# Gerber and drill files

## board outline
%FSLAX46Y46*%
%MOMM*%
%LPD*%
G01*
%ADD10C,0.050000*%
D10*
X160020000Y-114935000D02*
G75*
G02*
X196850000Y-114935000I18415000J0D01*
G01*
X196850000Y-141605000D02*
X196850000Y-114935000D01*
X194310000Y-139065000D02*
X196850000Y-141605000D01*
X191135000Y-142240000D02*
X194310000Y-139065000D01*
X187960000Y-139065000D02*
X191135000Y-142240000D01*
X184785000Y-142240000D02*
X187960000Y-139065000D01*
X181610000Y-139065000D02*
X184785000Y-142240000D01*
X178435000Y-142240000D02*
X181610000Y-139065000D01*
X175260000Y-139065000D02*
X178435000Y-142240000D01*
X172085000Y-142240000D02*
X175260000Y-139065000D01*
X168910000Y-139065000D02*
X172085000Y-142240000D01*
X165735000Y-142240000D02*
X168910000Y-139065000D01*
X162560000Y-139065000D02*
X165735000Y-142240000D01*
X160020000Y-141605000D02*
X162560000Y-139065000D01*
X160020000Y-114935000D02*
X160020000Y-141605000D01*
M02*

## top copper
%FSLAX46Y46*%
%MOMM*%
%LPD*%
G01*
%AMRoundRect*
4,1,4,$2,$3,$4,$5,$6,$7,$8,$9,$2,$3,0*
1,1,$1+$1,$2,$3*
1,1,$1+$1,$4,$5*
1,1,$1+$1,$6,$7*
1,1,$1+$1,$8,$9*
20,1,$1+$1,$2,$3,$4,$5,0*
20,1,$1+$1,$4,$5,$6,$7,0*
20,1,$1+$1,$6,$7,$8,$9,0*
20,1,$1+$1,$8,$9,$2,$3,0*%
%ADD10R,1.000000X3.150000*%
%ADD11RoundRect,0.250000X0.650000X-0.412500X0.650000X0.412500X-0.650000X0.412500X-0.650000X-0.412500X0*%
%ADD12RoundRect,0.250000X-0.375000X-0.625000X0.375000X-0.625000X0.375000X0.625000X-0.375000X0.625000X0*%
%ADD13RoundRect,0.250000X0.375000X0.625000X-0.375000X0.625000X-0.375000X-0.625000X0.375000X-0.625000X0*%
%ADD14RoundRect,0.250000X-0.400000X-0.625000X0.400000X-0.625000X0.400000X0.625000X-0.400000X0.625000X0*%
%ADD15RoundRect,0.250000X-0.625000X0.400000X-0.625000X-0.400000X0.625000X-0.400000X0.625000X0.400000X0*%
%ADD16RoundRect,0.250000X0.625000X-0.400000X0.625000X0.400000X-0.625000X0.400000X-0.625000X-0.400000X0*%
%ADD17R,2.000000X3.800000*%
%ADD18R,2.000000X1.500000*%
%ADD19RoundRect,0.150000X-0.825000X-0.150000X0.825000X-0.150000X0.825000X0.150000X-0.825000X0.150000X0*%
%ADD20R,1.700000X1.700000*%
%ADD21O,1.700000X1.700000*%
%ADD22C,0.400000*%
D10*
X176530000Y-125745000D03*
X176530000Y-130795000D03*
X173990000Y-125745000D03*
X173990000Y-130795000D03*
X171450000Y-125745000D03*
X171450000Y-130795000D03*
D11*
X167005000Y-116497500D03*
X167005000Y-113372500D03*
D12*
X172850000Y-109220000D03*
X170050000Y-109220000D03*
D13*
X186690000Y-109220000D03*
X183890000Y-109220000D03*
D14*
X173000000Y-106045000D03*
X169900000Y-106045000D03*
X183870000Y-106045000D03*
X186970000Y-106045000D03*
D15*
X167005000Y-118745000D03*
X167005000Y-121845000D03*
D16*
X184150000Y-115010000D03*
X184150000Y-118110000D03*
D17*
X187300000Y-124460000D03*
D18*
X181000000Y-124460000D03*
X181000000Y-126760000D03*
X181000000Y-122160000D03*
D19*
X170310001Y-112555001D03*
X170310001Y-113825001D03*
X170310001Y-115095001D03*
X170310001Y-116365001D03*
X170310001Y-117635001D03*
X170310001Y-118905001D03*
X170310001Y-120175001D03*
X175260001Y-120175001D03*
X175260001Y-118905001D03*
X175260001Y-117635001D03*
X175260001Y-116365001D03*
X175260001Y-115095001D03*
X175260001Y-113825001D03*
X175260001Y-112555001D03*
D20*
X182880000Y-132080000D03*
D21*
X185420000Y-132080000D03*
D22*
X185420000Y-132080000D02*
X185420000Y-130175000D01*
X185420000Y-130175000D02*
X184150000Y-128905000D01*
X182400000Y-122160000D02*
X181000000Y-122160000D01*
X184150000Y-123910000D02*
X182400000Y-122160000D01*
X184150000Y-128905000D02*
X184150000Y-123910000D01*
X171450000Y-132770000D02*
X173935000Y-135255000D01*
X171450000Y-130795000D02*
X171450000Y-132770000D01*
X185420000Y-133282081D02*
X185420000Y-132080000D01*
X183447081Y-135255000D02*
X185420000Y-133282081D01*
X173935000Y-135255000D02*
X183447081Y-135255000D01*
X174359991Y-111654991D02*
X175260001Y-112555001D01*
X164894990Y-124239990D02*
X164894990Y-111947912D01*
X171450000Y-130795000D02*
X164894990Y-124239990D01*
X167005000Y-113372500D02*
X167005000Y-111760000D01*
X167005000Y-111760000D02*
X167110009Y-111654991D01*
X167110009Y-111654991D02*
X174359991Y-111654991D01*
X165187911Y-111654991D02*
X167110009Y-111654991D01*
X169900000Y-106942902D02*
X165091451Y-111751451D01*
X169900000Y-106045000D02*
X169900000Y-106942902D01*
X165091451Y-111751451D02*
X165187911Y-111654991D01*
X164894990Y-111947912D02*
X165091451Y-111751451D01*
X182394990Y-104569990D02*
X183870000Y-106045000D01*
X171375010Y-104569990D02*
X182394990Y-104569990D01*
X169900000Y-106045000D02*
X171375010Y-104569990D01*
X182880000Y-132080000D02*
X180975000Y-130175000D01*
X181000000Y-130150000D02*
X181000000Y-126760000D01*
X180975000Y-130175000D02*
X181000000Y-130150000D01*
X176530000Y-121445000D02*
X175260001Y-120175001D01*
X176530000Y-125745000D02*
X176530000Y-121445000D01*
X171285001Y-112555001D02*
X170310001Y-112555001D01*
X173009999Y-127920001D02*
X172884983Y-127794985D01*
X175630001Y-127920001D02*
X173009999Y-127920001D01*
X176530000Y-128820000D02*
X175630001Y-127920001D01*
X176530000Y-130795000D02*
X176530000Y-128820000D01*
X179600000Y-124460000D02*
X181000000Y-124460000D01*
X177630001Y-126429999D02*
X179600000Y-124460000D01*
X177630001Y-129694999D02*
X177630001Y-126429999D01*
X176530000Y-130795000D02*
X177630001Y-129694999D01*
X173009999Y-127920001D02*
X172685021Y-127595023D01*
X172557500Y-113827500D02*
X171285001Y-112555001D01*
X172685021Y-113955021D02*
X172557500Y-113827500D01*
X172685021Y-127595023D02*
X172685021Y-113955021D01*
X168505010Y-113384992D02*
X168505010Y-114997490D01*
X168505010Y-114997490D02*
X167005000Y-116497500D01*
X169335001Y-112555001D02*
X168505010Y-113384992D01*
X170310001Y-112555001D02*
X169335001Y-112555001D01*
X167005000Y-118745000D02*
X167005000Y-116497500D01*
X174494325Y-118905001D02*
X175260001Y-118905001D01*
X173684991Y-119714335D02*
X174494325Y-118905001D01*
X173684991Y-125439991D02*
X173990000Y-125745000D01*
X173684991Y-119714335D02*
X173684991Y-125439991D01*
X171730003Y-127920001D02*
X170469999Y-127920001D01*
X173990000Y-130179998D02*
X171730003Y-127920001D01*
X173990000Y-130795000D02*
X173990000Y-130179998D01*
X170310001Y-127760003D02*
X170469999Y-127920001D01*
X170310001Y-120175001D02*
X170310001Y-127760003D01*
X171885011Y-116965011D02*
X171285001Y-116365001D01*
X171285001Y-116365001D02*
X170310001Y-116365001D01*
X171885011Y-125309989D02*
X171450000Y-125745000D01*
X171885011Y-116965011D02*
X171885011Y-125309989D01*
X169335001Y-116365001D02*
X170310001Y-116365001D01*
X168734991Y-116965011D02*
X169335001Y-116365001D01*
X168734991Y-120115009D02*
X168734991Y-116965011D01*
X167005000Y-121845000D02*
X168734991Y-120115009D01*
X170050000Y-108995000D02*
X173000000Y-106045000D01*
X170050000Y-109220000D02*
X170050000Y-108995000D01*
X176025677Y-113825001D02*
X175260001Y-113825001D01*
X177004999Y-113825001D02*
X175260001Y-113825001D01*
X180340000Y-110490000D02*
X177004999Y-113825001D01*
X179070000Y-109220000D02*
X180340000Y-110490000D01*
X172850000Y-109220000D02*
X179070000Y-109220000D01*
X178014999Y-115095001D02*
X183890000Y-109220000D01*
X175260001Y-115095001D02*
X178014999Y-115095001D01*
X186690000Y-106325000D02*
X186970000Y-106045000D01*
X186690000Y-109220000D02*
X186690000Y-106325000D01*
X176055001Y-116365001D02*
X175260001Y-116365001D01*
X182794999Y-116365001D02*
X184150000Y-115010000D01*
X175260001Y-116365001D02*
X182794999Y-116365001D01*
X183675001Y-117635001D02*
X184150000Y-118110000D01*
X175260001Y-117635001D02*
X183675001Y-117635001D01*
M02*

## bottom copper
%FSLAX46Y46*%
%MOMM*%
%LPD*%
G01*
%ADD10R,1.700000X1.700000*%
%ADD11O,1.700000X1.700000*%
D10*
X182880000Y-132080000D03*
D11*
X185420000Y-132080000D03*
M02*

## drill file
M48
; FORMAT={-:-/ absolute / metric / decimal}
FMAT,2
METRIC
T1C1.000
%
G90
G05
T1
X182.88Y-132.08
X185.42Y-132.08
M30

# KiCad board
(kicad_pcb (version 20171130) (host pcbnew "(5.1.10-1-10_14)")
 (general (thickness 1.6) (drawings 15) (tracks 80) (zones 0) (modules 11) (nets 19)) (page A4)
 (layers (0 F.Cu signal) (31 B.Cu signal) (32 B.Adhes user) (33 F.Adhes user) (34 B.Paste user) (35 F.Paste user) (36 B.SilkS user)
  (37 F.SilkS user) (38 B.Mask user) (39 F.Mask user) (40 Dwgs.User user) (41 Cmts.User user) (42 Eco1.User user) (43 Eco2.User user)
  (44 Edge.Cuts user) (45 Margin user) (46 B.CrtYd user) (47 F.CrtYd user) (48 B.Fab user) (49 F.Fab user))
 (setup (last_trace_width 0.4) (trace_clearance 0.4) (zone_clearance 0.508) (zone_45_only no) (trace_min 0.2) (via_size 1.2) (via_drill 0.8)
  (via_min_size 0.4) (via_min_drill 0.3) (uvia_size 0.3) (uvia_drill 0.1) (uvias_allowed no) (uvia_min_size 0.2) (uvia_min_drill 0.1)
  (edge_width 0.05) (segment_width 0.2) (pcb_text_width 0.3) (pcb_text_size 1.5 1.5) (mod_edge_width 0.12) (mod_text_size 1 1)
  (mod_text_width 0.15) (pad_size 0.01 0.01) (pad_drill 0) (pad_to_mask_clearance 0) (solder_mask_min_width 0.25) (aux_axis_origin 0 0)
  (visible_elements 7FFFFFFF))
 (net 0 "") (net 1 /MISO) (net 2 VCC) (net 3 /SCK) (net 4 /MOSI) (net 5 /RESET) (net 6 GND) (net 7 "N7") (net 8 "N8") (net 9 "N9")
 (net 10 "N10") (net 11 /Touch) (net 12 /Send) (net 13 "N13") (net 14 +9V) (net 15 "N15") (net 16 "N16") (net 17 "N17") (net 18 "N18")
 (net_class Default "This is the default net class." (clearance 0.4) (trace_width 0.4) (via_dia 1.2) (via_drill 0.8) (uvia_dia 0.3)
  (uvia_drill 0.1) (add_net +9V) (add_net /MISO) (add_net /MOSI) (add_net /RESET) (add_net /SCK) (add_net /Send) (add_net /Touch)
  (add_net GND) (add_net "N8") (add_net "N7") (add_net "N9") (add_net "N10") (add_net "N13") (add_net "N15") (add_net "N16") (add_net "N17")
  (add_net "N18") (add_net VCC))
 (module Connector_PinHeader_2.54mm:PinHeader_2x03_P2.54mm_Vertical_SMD (layer F.Cu) (at 173.99 128.27 270)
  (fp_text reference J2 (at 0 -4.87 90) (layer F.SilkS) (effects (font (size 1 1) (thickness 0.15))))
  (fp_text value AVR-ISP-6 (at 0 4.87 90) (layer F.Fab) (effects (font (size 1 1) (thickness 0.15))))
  (pad 1 smd rect (at -2.525 -2.54 270) (size 3.15 1) (layers F.Cu F.Paste F.Mask) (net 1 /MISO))
  (pad 2 smd rect (at 2.525 -2.54 270) (size 3.15 1) (layers F.Cu F.Paste F.Mask) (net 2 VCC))
  (pad 3 smd rect (at -2.525 0 270) (size 3.15 1) (layers F.Cu F.Paste F.Mask) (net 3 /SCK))
  (pad 4 smd rect (at 2.525 0 270) (size 3.15 1) (layers F.Cu F.Paste F.Mask) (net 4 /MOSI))
  (pad 5 smd rect (at -2.525 2.54 270) (size 3.15 1) (layers F.Cu F.Paste F.Mask) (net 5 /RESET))
  (pad 6 smd rect (at 2.525 2.54 270) (size 3.15 1) (layers F.Cu F.Paste F.Mask) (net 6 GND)))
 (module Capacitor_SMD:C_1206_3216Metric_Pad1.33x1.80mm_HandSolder (layer F.Cu) (at 167.005 114.935 90)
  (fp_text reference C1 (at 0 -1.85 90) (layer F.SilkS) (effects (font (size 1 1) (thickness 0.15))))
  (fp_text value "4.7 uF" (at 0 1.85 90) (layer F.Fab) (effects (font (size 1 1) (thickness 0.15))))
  (pad 1 smd roundrect (at -1.5625 0 90) (size 1.325 1.8) (layers F.Cu F.Paste F.Mask) (roundrect_rratio 0.188679) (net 2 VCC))
  (pad 2 smd roundrect (at 1.5625 0 90) (size 1.325 1.8) (layers F.Cu F.Paste F.Mask) (roundrect_rratio 0.188679) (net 6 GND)))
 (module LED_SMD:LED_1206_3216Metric (layer F.Cu) (at 171.45 109.22)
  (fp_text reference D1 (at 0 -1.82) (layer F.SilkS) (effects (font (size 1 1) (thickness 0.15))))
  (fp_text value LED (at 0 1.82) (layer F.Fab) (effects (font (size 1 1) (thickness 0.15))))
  (pad 2 smd roundrect (at 1.4 0) (size 1.25 1.75) (layers F.Cu F.Paste F.Mask) (roundrect_rratio 0.2) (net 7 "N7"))
  (pad 1 smd roundrect (at -1.4 0) (size 1.25 1.75) (layers F.Cu F.Paste F.Mask) (roundrect_rratio 0.2) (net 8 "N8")))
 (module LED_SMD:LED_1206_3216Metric (layer F.Cu) (at 185.29 109.22 180)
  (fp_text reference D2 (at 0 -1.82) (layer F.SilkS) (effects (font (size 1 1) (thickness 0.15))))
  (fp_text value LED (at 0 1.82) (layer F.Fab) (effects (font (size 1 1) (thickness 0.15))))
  (pad 1 smd roundrect (at -1.4 0 180) (size 1.25 1.75) (layers F.Cu F.Paste F.Mask) (roundrect_rratio 0.2) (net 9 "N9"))
  (pad 2 smd roundrect (at 1.4 0 180) (size 1.25 1.75) (layers F.Cu F.Paste F.Mask) (roundrect_rratio 0.2) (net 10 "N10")))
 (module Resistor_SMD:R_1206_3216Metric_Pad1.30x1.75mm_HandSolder (layer F.Cu) (at 171.45 106.045)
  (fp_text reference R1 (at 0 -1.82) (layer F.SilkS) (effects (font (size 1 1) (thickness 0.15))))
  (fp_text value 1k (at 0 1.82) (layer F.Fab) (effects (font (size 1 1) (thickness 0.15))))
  (pad 2 smd roundrect (at 1.55 0) (size 1.3 1.75) (layers F.Cu F.Paste F.Mask) (roundrect_rratio 0.192308) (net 8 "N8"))
  (pad 1 smd roundrect (at -1.55 0) (size 1.3 1.75) (layers F.Cu F.Paste F.Mask) (roundrect_rratio 0.192308) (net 6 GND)))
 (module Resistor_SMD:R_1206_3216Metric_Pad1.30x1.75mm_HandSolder (layer F.Cu) (at 185.42 106.045)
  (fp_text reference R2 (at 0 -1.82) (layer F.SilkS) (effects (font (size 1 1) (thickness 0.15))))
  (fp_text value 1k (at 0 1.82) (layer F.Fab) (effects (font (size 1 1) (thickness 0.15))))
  (pad 1 smd roundrect (at -1.55 0) (size 1.3 1.75) (layers F.Cu F.Paste F.Mask) (roundrect_rratio 0.192308) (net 6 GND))
  (pad 2 smd roundrect (at 1.55 0) (size 1.3 1.75) (layers F.Cu F.Paste F.Mask) (roundrect_rratio 0.192308) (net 9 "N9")))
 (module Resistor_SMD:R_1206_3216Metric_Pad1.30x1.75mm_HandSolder (layer F.Cu) (at 167.005 120.295 270)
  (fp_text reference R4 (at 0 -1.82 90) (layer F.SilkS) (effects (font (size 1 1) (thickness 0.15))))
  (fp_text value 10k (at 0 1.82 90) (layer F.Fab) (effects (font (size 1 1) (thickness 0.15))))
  (pad 1 smd roundrect (at -1.55 0 270) (size 1.3 1.75) (layers F.Cu F.Paste F.Mask) (roundrect_rratio 0.192308) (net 2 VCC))
  (pad 2 smd roundrect (at 1.55 0 270) (size 1.3 1.75) (layers F.Cu F.Paste F.Mask) (roundrect_rratio 0.192308) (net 5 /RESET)))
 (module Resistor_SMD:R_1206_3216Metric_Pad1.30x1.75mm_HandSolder (layer F.Cu) (at 184.15 116.56 90)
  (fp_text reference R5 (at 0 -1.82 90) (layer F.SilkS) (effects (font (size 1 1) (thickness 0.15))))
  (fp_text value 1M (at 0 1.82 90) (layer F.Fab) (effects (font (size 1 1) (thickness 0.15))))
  (pad 2 smd roundrect (at 1.55 0 90) (size 1.3 1.75) (layers F.Cu F.Paste F.Mask) (roundrect_rratio 0.192308) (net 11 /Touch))
  (pad 1 smd roundrect (at -1.55 0 90) (size 1.3 1.75) (layers F.Cu F.Paste F.Mask) (roundrect_rratio 0.192308) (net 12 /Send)))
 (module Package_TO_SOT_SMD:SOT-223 (layer F.Cu) (at 184.15 124.46)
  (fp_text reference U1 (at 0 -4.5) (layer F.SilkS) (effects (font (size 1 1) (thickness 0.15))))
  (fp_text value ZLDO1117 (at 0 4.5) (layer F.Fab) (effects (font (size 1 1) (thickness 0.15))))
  (pad 4 smd rect (at 3.15 0) (size 2 3.8) (layers F.Cu F.Paste F.Mask) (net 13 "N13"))
  (pad 2 smd rect (at -3.15 0) (size 2 1.5) (layers F.Cu F.Paste F.Mask) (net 2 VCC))
  (pad 3 smd rect (at -3.15 2.3) (size 2 1.5) (layers F.Cu F.Paste F.Mask) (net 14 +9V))
  (pad 1 smd rect (at -3.15 -2.3) (size 2 1.5) (layers F.Cu F.Paste F.Mask) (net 6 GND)))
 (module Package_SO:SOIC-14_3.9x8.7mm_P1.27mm (layer F.Cu) (at 172.785001 116.365001)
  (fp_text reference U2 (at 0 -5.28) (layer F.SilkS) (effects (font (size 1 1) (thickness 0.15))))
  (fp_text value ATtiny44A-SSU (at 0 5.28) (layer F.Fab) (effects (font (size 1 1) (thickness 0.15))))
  (pad 1 smd roundrect (at -2.475 -3.81) (size 1.95 0.6) (layers F.Cu F.Paste F.Mask) (roundrect_rratio 0.25) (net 2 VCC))
  (pad 2 smd roundrect (at -2.475 -2.54) (size 1.95 0.6) (layers F.Cu F.Paste F.Mask) (roundrect_rratio 0.25) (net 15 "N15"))
  (pad 3 smd roundrect (at -2.475 -1.27) (size 1.95 0.6) (layers F.Cu F.Paste F.Mask) (roundrect_rratio 0.25) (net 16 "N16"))
  (pad 4 smd roundrect (at -2.475 0) (size 1.95 0.6) (layers F.Cu F.Paste F.Mask) (roundrect_rratio 0.25) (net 5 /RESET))
  (pad 5 smd roundrect (at -2.475 1.27) (size 1.95 0.6) (layers F.Cu F.Paste F.Mask) (roundrect_rratio 0.25) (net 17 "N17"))
  (pad 6 smd roundrect (at -2.475 2.54) (size 1.95 0.6) (layers F.Cu F.Paste F.Mask) (roundrect_rratio 0.25) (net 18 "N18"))
  (pad 7 smd roundrect (at -2.475 3.81) (size 1.95 0.6) (layers F.Cu F.Paste F.Mask) (roundrect_rratio 0.25) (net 4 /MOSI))
  (pad 8 smd roundrect (at 2.475 3.81) (size 1.95 0.6) (layers F.Cu F.Paste F.Mask) (roundrect_rratio 0.25) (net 1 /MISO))
  (pad 9 smd roundrect (at 2.475 2.54) (size 1.95 0.6) (layers F.Cu F.Paste F.Mask) (roundrect_rratio 0.25) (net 3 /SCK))
  (pad 10 smd roundrect (at 2.475 1.27) (size 1.95 0.6) (layers F.Cu F.Paste F.Mask) (roundrect_rratio 0.25) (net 12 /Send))
  (pad 11 smd roundrect (at 2.475 0) (size 1.95 0.6) (layers F.Cu F.Paste F.Mask) (roundrect_rratio 0.25) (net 11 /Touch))
  (pad 12 smd roundrect (at 2.475 -1.27) (size 1.95 0.6) (layers F.Cu F.Paste F.Mask) (roundrect_rratio 0.25) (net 10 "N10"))
  (pad 13 smd roundrect (at 2.475 -2.54) (size 1.95 0.6) (layers F.Cu F.Paste F.Mask) (roundrect_rratio 0.25) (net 7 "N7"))
  (pad 14 smd roundrect (at 2.475 -3.81) (size 1.95 0.6) (layers F.Cu F.Paste F.Mask) (roundrect_rratio 0.25) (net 6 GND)))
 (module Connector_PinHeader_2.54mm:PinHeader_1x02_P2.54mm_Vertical (layer F.Cu) (at 182.88 132.08 90)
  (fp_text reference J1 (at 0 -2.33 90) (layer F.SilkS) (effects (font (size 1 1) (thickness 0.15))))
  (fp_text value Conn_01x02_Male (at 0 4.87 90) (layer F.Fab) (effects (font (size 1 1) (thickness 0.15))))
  (pad 1 thru_hole rect (at 0 0 90) (size 1.7 1.7) (drill 1) (layers *.Cu *.Mask) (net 14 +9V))
  (pad 2 thru_hole oval (at 0 2.54 90) (size 1.7 1.7) (drill 1) (layers *.Cu *.Mask) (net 6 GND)))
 (gr_arc (start 178.435 114.935) (end 196.85 114.935) (angle -180) (layer Edge.Cuts) (width 0.05))
 (gr_line (start 196.85 141.605) (end 196.85 114.935) (layer Edge.Cuts) (width 0.05))
 (gr_line (start 194.31 139.065) (end 196.85 141.605) (layer Edge.Cuts) (width 0.05))
 (gr_line (start 191.135 142.24) (end 194.31 139.065) (layer Edge.Cuts) (width 0.05))
 (gr_line (start 187.96 139.065) (end 191.135 142.24) (layer Edge.Cuts) (width 0.05))
 (gr_line (start 184.785 142.24) (end 187.96 139.065) (layer Edge.Cuts) (width 0.05))
 (gr_line (start 181.61 139.065) (end 184.785 142.24) (layer Edge.Cuts) (width 0.05))
 (gr_line (start 178.435 142.24) (end 181.61 139.065) (layer Edge.Cuts) (width 0.05))
 (gr_line (start 175.26 139.065) (end 178.435 142.24) (layer Edge.Cuts) (width 0.05))
 (gr_line (start 172.085 142.24) (end 175.26 139.065) (layer Edge.Cuts) (width 0.05))
 (gr_line (start 168.91 139.065) (end 172.085 142.24) (layer Edge.Cuts) (width 0.05))
 (gr_line (start 165.735 142.24) (end 168.91 139.065) (layer Edge.Cuts) (width 0.05))
 (gr_line (start 162.56 139.065) (end 165.735 142.24) (layer Edge.Cuts) (width 0.05))
 (gr_line (start 160.02 141.605) (end 162.56 139.065) (layer Edge.Cuts) (width 0.05))
 (gr_line (start 160.02 114.935) (end 160.02 141.605) (layer Edge.Cuts) (width 0.05))
 (segment (start 185.42 132.08) (end 185.42 130.175) (width 0.4) (layer F.Cu) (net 6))
 (segment (start 185.42 130.175) (end 184.15 128.905) (width 0.4) (layer F.Cu) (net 6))
 (segment (start 182.4 122.16) (end 181 122.16) (width 0.4) (layer F.Cu) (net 6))
 (segment (start 184.15 123.91) (end 182.4 122.16) (width 0.4) (layer F.Cu) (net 6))
 (segment (start 184.15 128.905) (end 184.15 123.91) (width 0.4) (layer F.Cu) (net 6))
 (segment (start 171.45 132.77) (end 173.935 135.255) (width 0.4) (layer F.Cu) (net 6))
 (segment (start 171.45 130.795) (end 171.45 132.77) (width 0.4) (layer F.Cu) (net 6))
 (segment (start 185.42 133.282081) (end 185.42 132.08) (width 0.4) (layer F.Cu) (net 6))
 (segment (start 183.447081 135.255) (end 185.42 133.282081) (width 0.4) (layer F.Cu) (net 6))
 (segment (start 173.935 135.255) (end 183.447081 135.255) (width 0.4) (layer F.Cu) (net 6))
 (segment (start 174.359991 111.654991) (end 175.260001 112.555001) (width 0.4) (layer F.Cu) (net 6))
 (segment (start 164.89499 124.23999) (end 164.89499 111.947912) (width 0.4) (layer F.Cu) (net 6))
 (segment (start 171.45 130.795) (end 164.89499 124.23999) (width 0.4) (layer F.Cu) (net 6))
 (segment (start 167.005 113.3725) (end 167.005 111.76) (width 0.4) (layer F.Cu) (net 6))
 (segment (start 167.005 111.76) (end 167.110009 111.654991) (width 0.4) (layer F.Cu) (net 6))
 (segment (start 167.110009 111.654991) (end 174.359991 111.654991) (width 0.4) (layer F.Cu) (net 6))
 (segment (start 165.187911 111.654991) (end 167.110009 111.654991) (width 0.4) (layer F.Cu) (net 6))
 (segment (start 169.9 106.942902) (end 165.091451 111.751451) (width 0.4) (layer F.Cu) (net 6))
 (segment (start 169.9 106.045) (end 169.9 106.942902) (width 0.4) (layer F.Cu) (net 6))
 (segment (start 165.091451 111.751451) (end 165.187911 111.654991) (width 0.4) (layer F.Cu) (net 6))
 (segment (start 164.89499 111.947912) (end 165.091451 111.751451) (width 0.4) (layer F.Cu) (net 6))
 (segment (start 182.39499 104.56999) (end 183.87 106.045) (width 0.4) (layer F.Cu) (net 6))
 (segment (start 171.37501 104.56999) (end 182.39499 104.56999) (width 0.4) (layer F.Cu) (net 6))
 (segment (start 169.9 106.045) (end 171.37501 104.56999) (width 0.4) (layer F.Cu) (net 6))
 (segment (start 182.88 132.08) (end 180.975 130.175) (width 0.4) (layer F.Cu) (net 14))
 (segment (start 181 130.15) (end 181 126.76) (width 0.4) (layer F.Cu) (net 14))
 (segment (start 180.975 130.175) (end 181 130.15) (width 0.4) (layer F.Cu) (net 14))
 (segment (start 176.53 121.445) (end 175.260001 120.175001) (width 0.4) (layer F.Cu) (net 1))
 (segment (start 176.53 125.745) (end 176.53 121.445) (width 0.4) (layer F.Cu) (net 1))
 (segment (start 171.285001 112.555001) (end 170.310001 112.555001) (width 0.4) (layer F.Cu) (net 2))
 (segment (start 173.009999 127.920001) (end 172.884983 127.794985) (width 0.4) (layer F.Cu) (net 2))
 (segment (start 175.630001 127.920001) (end 173.009999 127.920001) (width 0.4) (layer F.Cu) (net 2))
 (segment (start 176.53 128.82) (end 175.630001 127.920001) (width 0.4) (layer F.Cu) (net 2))
 (segment (start 176.53 130.795) (end 176.53 128.82) (width 0.4) (layer F.Cu) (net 2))
 (segment (start 179.6 124.46) (end 181 124.46) (width 0.4) (layer F.Cu) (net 2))
 (segment (start 177.630001 126.429999) (end 179.6 124.46) (width 0.4) (layer F.Cu) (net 2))
 (segment (start 177.630001 129.694999) (end 177.630001 126.429999) (width 0.4) (layer F.Cu) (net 2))
 (segment (start 176.53 130.795) (end 177.630001 129.694999) (width 0.4) (layer F.Cu) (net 2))
 (segment (start 173.009999 127.920001) (end 172.685021 127.595023) (width 0.4) (layer F.Cu) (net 2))
 (segment (start 172.5575 113.8275) (end 171.285001 112.555001) (width 0.4) (layer F.Cu) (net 2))
 (segment (start 172.685021 113.955021) (end 172.5575 113.8275) (width 0.4) (layer F.Cu) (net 2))
 (segment (start 172.685021 127.595023) (end 172.685021 113.955021) (width 0.4) (layer F.Cu) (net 2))
 (segment (start 168.50501 113.384992) (end 168.50501 114.99749) (width 0.4) (layer F.Cu) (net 2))
 (segment (start 168.50501 114.99749) (end 167.005 116.4975) (width 0.4) (layer F.Cu) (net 2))
 (segment (start 169.335001 112.555001) (end 168.50501 113.384992) (width 0.4) (layer F.Cu) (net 2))
 (segment (start 170.310001 112.555001) (end 169.335001 112.555001) (width 0.4) (layer F.Cu) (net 2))
 (segment (start 167.005 118.745) (end 167.005 116.4975) (width 0.4) (layer F.Cu) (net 2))
 (segment (start 174.494325 118.905001) (end 175.260001 118.905001) (width 0.4) (layer F.Cu) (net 3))
 (segment (start 173.684991 119.714335) (end 174.494325 118.905001) (width 0.4) (layer F.Cu) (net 3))
 (segment (start 173.684991 125.439991) (end 173.99 125.745) (width 0.4) (layer F.Cu) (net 3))
 (segment (start 173.684991 119.714335) (end 173.684991 125.439991) (width 0.4) (layer F.Cu) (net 3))
 (segment (start 171.730003 127.920001) (end 170.469999 127.920001) (width 0.4) (layer F.Cu) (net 4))
 (segment (start 173.99 130.179998) (end 171.730003 127.920001) (width 0.4) (layer F.Cu) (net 4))
 (segment (start 173.99 130.795) (end 173.99 130.179998) (width 0.4) (layer F.Cu) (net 4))
 (segment (start 170.310001 127.760003) (end 170.469999 127.920001) (width 0.4) (layer F.Cu) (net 4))
 (segment (start 170.310001 120.175001) (end 170.310001 127.760003) (width 0.4) (layer F.Cu) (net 4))
 (segment (start 171.885011 116.965011) (end 171.285001 116.365001) (width 0.4) (layer F.Cu) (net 5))
 (segment (start 171.285001 116.365001) (end 170.310001 116.365001) (width 0.4) (layer F.Cu) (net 5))
 (segment (start 171.885011 125.309989) (end 171.45 125.745) (width 0.4) (layer F.Cu) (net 5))
 (segment (start 171.885011 116.965011) (end 171.885011 125.309989) (width 0.4) (layer F.Cu) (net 5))
 (segment (start 169.335001 116.365001) (end 170.310001 116.365001) (width 0.4) (layer F.Cu) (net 5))
 (segment (start 168.734991 116.965011) (end 169.335001 116.365001) (width 0.4) (layer F.Cu) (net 5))
 (segment (start 168.734991 120.115009) (end 168.734991 116.965011) (width 0.4) (layer F.Cu) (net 5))
 (segment (start 167.005 121.845) (end 168.734991 120.115009) (width 0.4) (layer F.Cu) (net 5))
 (segment (start 170.05 108.995) (end 173 106.045) (width 0.4) (layer F.Cu) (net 8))
 (segment (start 170.05 109.22) (end 170.05 108.995) (width 0.4) (layer F.Cu) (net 8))
 (segment (start 176.025677 113.825001) (end 175.260001 113.825001) (width 0.4) (layer F.Cu) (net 7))
 (segment (start 177.004999 113.825001) (end 175.260001 113.825001) (width 0.4) (layer F.Cu) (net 7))
 (segment (start 180.34 110.49) (end 177.004999 113.825001) (width 0.4) (layer F.Cu) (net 7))
 (segment (start 179.07 109.22) (end 180.34 110.49) (width 0.4) (layer F.Cu) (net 7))
 (segment (start 172.85 109.22) (end 179.07 109.22) (width 0.4) (layer F.Cu) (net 7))
 (segment (start 178.014999 115.095001) (end 183.89 109.22) (width 0.4) (layer F.Cu) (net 10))
 (segment (start 175.260001 115.095001) (end 178.014999 115.095001) (width 0.4) (layer F.Cu) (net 10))
 (segment (start 186.69 106.325) (end 186.97 106.045) (width 0.4) (layer F.Cu) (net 9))
 (segment (start 186.69 109.22) (end 186.69 106.325) (width 0.4) (layer F.Cu) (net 9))
 (segment (start 176.055001 116.365001) (end 175.260001 116.365001) (width 0.4) (layer F.Cu) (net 11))
 (segment (start 182.794999 116.365001) (end 184.15 115.01) (width 0.4) (layer F.Cu) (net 11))
 (segment (start 175.260001 116.365001) (end 182.794999 116.365001) (width 0.4) (layer F.Cu) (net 11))
 (segment (start 183.675001 117.635001) (end 184.15 118.11) (width 0.4) (layer F.Cu) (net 12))
 (segment (start 175.260001 117.635001) (end 183.675001 117.635001) (width 0.4) (layer F.Cu) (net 12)))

